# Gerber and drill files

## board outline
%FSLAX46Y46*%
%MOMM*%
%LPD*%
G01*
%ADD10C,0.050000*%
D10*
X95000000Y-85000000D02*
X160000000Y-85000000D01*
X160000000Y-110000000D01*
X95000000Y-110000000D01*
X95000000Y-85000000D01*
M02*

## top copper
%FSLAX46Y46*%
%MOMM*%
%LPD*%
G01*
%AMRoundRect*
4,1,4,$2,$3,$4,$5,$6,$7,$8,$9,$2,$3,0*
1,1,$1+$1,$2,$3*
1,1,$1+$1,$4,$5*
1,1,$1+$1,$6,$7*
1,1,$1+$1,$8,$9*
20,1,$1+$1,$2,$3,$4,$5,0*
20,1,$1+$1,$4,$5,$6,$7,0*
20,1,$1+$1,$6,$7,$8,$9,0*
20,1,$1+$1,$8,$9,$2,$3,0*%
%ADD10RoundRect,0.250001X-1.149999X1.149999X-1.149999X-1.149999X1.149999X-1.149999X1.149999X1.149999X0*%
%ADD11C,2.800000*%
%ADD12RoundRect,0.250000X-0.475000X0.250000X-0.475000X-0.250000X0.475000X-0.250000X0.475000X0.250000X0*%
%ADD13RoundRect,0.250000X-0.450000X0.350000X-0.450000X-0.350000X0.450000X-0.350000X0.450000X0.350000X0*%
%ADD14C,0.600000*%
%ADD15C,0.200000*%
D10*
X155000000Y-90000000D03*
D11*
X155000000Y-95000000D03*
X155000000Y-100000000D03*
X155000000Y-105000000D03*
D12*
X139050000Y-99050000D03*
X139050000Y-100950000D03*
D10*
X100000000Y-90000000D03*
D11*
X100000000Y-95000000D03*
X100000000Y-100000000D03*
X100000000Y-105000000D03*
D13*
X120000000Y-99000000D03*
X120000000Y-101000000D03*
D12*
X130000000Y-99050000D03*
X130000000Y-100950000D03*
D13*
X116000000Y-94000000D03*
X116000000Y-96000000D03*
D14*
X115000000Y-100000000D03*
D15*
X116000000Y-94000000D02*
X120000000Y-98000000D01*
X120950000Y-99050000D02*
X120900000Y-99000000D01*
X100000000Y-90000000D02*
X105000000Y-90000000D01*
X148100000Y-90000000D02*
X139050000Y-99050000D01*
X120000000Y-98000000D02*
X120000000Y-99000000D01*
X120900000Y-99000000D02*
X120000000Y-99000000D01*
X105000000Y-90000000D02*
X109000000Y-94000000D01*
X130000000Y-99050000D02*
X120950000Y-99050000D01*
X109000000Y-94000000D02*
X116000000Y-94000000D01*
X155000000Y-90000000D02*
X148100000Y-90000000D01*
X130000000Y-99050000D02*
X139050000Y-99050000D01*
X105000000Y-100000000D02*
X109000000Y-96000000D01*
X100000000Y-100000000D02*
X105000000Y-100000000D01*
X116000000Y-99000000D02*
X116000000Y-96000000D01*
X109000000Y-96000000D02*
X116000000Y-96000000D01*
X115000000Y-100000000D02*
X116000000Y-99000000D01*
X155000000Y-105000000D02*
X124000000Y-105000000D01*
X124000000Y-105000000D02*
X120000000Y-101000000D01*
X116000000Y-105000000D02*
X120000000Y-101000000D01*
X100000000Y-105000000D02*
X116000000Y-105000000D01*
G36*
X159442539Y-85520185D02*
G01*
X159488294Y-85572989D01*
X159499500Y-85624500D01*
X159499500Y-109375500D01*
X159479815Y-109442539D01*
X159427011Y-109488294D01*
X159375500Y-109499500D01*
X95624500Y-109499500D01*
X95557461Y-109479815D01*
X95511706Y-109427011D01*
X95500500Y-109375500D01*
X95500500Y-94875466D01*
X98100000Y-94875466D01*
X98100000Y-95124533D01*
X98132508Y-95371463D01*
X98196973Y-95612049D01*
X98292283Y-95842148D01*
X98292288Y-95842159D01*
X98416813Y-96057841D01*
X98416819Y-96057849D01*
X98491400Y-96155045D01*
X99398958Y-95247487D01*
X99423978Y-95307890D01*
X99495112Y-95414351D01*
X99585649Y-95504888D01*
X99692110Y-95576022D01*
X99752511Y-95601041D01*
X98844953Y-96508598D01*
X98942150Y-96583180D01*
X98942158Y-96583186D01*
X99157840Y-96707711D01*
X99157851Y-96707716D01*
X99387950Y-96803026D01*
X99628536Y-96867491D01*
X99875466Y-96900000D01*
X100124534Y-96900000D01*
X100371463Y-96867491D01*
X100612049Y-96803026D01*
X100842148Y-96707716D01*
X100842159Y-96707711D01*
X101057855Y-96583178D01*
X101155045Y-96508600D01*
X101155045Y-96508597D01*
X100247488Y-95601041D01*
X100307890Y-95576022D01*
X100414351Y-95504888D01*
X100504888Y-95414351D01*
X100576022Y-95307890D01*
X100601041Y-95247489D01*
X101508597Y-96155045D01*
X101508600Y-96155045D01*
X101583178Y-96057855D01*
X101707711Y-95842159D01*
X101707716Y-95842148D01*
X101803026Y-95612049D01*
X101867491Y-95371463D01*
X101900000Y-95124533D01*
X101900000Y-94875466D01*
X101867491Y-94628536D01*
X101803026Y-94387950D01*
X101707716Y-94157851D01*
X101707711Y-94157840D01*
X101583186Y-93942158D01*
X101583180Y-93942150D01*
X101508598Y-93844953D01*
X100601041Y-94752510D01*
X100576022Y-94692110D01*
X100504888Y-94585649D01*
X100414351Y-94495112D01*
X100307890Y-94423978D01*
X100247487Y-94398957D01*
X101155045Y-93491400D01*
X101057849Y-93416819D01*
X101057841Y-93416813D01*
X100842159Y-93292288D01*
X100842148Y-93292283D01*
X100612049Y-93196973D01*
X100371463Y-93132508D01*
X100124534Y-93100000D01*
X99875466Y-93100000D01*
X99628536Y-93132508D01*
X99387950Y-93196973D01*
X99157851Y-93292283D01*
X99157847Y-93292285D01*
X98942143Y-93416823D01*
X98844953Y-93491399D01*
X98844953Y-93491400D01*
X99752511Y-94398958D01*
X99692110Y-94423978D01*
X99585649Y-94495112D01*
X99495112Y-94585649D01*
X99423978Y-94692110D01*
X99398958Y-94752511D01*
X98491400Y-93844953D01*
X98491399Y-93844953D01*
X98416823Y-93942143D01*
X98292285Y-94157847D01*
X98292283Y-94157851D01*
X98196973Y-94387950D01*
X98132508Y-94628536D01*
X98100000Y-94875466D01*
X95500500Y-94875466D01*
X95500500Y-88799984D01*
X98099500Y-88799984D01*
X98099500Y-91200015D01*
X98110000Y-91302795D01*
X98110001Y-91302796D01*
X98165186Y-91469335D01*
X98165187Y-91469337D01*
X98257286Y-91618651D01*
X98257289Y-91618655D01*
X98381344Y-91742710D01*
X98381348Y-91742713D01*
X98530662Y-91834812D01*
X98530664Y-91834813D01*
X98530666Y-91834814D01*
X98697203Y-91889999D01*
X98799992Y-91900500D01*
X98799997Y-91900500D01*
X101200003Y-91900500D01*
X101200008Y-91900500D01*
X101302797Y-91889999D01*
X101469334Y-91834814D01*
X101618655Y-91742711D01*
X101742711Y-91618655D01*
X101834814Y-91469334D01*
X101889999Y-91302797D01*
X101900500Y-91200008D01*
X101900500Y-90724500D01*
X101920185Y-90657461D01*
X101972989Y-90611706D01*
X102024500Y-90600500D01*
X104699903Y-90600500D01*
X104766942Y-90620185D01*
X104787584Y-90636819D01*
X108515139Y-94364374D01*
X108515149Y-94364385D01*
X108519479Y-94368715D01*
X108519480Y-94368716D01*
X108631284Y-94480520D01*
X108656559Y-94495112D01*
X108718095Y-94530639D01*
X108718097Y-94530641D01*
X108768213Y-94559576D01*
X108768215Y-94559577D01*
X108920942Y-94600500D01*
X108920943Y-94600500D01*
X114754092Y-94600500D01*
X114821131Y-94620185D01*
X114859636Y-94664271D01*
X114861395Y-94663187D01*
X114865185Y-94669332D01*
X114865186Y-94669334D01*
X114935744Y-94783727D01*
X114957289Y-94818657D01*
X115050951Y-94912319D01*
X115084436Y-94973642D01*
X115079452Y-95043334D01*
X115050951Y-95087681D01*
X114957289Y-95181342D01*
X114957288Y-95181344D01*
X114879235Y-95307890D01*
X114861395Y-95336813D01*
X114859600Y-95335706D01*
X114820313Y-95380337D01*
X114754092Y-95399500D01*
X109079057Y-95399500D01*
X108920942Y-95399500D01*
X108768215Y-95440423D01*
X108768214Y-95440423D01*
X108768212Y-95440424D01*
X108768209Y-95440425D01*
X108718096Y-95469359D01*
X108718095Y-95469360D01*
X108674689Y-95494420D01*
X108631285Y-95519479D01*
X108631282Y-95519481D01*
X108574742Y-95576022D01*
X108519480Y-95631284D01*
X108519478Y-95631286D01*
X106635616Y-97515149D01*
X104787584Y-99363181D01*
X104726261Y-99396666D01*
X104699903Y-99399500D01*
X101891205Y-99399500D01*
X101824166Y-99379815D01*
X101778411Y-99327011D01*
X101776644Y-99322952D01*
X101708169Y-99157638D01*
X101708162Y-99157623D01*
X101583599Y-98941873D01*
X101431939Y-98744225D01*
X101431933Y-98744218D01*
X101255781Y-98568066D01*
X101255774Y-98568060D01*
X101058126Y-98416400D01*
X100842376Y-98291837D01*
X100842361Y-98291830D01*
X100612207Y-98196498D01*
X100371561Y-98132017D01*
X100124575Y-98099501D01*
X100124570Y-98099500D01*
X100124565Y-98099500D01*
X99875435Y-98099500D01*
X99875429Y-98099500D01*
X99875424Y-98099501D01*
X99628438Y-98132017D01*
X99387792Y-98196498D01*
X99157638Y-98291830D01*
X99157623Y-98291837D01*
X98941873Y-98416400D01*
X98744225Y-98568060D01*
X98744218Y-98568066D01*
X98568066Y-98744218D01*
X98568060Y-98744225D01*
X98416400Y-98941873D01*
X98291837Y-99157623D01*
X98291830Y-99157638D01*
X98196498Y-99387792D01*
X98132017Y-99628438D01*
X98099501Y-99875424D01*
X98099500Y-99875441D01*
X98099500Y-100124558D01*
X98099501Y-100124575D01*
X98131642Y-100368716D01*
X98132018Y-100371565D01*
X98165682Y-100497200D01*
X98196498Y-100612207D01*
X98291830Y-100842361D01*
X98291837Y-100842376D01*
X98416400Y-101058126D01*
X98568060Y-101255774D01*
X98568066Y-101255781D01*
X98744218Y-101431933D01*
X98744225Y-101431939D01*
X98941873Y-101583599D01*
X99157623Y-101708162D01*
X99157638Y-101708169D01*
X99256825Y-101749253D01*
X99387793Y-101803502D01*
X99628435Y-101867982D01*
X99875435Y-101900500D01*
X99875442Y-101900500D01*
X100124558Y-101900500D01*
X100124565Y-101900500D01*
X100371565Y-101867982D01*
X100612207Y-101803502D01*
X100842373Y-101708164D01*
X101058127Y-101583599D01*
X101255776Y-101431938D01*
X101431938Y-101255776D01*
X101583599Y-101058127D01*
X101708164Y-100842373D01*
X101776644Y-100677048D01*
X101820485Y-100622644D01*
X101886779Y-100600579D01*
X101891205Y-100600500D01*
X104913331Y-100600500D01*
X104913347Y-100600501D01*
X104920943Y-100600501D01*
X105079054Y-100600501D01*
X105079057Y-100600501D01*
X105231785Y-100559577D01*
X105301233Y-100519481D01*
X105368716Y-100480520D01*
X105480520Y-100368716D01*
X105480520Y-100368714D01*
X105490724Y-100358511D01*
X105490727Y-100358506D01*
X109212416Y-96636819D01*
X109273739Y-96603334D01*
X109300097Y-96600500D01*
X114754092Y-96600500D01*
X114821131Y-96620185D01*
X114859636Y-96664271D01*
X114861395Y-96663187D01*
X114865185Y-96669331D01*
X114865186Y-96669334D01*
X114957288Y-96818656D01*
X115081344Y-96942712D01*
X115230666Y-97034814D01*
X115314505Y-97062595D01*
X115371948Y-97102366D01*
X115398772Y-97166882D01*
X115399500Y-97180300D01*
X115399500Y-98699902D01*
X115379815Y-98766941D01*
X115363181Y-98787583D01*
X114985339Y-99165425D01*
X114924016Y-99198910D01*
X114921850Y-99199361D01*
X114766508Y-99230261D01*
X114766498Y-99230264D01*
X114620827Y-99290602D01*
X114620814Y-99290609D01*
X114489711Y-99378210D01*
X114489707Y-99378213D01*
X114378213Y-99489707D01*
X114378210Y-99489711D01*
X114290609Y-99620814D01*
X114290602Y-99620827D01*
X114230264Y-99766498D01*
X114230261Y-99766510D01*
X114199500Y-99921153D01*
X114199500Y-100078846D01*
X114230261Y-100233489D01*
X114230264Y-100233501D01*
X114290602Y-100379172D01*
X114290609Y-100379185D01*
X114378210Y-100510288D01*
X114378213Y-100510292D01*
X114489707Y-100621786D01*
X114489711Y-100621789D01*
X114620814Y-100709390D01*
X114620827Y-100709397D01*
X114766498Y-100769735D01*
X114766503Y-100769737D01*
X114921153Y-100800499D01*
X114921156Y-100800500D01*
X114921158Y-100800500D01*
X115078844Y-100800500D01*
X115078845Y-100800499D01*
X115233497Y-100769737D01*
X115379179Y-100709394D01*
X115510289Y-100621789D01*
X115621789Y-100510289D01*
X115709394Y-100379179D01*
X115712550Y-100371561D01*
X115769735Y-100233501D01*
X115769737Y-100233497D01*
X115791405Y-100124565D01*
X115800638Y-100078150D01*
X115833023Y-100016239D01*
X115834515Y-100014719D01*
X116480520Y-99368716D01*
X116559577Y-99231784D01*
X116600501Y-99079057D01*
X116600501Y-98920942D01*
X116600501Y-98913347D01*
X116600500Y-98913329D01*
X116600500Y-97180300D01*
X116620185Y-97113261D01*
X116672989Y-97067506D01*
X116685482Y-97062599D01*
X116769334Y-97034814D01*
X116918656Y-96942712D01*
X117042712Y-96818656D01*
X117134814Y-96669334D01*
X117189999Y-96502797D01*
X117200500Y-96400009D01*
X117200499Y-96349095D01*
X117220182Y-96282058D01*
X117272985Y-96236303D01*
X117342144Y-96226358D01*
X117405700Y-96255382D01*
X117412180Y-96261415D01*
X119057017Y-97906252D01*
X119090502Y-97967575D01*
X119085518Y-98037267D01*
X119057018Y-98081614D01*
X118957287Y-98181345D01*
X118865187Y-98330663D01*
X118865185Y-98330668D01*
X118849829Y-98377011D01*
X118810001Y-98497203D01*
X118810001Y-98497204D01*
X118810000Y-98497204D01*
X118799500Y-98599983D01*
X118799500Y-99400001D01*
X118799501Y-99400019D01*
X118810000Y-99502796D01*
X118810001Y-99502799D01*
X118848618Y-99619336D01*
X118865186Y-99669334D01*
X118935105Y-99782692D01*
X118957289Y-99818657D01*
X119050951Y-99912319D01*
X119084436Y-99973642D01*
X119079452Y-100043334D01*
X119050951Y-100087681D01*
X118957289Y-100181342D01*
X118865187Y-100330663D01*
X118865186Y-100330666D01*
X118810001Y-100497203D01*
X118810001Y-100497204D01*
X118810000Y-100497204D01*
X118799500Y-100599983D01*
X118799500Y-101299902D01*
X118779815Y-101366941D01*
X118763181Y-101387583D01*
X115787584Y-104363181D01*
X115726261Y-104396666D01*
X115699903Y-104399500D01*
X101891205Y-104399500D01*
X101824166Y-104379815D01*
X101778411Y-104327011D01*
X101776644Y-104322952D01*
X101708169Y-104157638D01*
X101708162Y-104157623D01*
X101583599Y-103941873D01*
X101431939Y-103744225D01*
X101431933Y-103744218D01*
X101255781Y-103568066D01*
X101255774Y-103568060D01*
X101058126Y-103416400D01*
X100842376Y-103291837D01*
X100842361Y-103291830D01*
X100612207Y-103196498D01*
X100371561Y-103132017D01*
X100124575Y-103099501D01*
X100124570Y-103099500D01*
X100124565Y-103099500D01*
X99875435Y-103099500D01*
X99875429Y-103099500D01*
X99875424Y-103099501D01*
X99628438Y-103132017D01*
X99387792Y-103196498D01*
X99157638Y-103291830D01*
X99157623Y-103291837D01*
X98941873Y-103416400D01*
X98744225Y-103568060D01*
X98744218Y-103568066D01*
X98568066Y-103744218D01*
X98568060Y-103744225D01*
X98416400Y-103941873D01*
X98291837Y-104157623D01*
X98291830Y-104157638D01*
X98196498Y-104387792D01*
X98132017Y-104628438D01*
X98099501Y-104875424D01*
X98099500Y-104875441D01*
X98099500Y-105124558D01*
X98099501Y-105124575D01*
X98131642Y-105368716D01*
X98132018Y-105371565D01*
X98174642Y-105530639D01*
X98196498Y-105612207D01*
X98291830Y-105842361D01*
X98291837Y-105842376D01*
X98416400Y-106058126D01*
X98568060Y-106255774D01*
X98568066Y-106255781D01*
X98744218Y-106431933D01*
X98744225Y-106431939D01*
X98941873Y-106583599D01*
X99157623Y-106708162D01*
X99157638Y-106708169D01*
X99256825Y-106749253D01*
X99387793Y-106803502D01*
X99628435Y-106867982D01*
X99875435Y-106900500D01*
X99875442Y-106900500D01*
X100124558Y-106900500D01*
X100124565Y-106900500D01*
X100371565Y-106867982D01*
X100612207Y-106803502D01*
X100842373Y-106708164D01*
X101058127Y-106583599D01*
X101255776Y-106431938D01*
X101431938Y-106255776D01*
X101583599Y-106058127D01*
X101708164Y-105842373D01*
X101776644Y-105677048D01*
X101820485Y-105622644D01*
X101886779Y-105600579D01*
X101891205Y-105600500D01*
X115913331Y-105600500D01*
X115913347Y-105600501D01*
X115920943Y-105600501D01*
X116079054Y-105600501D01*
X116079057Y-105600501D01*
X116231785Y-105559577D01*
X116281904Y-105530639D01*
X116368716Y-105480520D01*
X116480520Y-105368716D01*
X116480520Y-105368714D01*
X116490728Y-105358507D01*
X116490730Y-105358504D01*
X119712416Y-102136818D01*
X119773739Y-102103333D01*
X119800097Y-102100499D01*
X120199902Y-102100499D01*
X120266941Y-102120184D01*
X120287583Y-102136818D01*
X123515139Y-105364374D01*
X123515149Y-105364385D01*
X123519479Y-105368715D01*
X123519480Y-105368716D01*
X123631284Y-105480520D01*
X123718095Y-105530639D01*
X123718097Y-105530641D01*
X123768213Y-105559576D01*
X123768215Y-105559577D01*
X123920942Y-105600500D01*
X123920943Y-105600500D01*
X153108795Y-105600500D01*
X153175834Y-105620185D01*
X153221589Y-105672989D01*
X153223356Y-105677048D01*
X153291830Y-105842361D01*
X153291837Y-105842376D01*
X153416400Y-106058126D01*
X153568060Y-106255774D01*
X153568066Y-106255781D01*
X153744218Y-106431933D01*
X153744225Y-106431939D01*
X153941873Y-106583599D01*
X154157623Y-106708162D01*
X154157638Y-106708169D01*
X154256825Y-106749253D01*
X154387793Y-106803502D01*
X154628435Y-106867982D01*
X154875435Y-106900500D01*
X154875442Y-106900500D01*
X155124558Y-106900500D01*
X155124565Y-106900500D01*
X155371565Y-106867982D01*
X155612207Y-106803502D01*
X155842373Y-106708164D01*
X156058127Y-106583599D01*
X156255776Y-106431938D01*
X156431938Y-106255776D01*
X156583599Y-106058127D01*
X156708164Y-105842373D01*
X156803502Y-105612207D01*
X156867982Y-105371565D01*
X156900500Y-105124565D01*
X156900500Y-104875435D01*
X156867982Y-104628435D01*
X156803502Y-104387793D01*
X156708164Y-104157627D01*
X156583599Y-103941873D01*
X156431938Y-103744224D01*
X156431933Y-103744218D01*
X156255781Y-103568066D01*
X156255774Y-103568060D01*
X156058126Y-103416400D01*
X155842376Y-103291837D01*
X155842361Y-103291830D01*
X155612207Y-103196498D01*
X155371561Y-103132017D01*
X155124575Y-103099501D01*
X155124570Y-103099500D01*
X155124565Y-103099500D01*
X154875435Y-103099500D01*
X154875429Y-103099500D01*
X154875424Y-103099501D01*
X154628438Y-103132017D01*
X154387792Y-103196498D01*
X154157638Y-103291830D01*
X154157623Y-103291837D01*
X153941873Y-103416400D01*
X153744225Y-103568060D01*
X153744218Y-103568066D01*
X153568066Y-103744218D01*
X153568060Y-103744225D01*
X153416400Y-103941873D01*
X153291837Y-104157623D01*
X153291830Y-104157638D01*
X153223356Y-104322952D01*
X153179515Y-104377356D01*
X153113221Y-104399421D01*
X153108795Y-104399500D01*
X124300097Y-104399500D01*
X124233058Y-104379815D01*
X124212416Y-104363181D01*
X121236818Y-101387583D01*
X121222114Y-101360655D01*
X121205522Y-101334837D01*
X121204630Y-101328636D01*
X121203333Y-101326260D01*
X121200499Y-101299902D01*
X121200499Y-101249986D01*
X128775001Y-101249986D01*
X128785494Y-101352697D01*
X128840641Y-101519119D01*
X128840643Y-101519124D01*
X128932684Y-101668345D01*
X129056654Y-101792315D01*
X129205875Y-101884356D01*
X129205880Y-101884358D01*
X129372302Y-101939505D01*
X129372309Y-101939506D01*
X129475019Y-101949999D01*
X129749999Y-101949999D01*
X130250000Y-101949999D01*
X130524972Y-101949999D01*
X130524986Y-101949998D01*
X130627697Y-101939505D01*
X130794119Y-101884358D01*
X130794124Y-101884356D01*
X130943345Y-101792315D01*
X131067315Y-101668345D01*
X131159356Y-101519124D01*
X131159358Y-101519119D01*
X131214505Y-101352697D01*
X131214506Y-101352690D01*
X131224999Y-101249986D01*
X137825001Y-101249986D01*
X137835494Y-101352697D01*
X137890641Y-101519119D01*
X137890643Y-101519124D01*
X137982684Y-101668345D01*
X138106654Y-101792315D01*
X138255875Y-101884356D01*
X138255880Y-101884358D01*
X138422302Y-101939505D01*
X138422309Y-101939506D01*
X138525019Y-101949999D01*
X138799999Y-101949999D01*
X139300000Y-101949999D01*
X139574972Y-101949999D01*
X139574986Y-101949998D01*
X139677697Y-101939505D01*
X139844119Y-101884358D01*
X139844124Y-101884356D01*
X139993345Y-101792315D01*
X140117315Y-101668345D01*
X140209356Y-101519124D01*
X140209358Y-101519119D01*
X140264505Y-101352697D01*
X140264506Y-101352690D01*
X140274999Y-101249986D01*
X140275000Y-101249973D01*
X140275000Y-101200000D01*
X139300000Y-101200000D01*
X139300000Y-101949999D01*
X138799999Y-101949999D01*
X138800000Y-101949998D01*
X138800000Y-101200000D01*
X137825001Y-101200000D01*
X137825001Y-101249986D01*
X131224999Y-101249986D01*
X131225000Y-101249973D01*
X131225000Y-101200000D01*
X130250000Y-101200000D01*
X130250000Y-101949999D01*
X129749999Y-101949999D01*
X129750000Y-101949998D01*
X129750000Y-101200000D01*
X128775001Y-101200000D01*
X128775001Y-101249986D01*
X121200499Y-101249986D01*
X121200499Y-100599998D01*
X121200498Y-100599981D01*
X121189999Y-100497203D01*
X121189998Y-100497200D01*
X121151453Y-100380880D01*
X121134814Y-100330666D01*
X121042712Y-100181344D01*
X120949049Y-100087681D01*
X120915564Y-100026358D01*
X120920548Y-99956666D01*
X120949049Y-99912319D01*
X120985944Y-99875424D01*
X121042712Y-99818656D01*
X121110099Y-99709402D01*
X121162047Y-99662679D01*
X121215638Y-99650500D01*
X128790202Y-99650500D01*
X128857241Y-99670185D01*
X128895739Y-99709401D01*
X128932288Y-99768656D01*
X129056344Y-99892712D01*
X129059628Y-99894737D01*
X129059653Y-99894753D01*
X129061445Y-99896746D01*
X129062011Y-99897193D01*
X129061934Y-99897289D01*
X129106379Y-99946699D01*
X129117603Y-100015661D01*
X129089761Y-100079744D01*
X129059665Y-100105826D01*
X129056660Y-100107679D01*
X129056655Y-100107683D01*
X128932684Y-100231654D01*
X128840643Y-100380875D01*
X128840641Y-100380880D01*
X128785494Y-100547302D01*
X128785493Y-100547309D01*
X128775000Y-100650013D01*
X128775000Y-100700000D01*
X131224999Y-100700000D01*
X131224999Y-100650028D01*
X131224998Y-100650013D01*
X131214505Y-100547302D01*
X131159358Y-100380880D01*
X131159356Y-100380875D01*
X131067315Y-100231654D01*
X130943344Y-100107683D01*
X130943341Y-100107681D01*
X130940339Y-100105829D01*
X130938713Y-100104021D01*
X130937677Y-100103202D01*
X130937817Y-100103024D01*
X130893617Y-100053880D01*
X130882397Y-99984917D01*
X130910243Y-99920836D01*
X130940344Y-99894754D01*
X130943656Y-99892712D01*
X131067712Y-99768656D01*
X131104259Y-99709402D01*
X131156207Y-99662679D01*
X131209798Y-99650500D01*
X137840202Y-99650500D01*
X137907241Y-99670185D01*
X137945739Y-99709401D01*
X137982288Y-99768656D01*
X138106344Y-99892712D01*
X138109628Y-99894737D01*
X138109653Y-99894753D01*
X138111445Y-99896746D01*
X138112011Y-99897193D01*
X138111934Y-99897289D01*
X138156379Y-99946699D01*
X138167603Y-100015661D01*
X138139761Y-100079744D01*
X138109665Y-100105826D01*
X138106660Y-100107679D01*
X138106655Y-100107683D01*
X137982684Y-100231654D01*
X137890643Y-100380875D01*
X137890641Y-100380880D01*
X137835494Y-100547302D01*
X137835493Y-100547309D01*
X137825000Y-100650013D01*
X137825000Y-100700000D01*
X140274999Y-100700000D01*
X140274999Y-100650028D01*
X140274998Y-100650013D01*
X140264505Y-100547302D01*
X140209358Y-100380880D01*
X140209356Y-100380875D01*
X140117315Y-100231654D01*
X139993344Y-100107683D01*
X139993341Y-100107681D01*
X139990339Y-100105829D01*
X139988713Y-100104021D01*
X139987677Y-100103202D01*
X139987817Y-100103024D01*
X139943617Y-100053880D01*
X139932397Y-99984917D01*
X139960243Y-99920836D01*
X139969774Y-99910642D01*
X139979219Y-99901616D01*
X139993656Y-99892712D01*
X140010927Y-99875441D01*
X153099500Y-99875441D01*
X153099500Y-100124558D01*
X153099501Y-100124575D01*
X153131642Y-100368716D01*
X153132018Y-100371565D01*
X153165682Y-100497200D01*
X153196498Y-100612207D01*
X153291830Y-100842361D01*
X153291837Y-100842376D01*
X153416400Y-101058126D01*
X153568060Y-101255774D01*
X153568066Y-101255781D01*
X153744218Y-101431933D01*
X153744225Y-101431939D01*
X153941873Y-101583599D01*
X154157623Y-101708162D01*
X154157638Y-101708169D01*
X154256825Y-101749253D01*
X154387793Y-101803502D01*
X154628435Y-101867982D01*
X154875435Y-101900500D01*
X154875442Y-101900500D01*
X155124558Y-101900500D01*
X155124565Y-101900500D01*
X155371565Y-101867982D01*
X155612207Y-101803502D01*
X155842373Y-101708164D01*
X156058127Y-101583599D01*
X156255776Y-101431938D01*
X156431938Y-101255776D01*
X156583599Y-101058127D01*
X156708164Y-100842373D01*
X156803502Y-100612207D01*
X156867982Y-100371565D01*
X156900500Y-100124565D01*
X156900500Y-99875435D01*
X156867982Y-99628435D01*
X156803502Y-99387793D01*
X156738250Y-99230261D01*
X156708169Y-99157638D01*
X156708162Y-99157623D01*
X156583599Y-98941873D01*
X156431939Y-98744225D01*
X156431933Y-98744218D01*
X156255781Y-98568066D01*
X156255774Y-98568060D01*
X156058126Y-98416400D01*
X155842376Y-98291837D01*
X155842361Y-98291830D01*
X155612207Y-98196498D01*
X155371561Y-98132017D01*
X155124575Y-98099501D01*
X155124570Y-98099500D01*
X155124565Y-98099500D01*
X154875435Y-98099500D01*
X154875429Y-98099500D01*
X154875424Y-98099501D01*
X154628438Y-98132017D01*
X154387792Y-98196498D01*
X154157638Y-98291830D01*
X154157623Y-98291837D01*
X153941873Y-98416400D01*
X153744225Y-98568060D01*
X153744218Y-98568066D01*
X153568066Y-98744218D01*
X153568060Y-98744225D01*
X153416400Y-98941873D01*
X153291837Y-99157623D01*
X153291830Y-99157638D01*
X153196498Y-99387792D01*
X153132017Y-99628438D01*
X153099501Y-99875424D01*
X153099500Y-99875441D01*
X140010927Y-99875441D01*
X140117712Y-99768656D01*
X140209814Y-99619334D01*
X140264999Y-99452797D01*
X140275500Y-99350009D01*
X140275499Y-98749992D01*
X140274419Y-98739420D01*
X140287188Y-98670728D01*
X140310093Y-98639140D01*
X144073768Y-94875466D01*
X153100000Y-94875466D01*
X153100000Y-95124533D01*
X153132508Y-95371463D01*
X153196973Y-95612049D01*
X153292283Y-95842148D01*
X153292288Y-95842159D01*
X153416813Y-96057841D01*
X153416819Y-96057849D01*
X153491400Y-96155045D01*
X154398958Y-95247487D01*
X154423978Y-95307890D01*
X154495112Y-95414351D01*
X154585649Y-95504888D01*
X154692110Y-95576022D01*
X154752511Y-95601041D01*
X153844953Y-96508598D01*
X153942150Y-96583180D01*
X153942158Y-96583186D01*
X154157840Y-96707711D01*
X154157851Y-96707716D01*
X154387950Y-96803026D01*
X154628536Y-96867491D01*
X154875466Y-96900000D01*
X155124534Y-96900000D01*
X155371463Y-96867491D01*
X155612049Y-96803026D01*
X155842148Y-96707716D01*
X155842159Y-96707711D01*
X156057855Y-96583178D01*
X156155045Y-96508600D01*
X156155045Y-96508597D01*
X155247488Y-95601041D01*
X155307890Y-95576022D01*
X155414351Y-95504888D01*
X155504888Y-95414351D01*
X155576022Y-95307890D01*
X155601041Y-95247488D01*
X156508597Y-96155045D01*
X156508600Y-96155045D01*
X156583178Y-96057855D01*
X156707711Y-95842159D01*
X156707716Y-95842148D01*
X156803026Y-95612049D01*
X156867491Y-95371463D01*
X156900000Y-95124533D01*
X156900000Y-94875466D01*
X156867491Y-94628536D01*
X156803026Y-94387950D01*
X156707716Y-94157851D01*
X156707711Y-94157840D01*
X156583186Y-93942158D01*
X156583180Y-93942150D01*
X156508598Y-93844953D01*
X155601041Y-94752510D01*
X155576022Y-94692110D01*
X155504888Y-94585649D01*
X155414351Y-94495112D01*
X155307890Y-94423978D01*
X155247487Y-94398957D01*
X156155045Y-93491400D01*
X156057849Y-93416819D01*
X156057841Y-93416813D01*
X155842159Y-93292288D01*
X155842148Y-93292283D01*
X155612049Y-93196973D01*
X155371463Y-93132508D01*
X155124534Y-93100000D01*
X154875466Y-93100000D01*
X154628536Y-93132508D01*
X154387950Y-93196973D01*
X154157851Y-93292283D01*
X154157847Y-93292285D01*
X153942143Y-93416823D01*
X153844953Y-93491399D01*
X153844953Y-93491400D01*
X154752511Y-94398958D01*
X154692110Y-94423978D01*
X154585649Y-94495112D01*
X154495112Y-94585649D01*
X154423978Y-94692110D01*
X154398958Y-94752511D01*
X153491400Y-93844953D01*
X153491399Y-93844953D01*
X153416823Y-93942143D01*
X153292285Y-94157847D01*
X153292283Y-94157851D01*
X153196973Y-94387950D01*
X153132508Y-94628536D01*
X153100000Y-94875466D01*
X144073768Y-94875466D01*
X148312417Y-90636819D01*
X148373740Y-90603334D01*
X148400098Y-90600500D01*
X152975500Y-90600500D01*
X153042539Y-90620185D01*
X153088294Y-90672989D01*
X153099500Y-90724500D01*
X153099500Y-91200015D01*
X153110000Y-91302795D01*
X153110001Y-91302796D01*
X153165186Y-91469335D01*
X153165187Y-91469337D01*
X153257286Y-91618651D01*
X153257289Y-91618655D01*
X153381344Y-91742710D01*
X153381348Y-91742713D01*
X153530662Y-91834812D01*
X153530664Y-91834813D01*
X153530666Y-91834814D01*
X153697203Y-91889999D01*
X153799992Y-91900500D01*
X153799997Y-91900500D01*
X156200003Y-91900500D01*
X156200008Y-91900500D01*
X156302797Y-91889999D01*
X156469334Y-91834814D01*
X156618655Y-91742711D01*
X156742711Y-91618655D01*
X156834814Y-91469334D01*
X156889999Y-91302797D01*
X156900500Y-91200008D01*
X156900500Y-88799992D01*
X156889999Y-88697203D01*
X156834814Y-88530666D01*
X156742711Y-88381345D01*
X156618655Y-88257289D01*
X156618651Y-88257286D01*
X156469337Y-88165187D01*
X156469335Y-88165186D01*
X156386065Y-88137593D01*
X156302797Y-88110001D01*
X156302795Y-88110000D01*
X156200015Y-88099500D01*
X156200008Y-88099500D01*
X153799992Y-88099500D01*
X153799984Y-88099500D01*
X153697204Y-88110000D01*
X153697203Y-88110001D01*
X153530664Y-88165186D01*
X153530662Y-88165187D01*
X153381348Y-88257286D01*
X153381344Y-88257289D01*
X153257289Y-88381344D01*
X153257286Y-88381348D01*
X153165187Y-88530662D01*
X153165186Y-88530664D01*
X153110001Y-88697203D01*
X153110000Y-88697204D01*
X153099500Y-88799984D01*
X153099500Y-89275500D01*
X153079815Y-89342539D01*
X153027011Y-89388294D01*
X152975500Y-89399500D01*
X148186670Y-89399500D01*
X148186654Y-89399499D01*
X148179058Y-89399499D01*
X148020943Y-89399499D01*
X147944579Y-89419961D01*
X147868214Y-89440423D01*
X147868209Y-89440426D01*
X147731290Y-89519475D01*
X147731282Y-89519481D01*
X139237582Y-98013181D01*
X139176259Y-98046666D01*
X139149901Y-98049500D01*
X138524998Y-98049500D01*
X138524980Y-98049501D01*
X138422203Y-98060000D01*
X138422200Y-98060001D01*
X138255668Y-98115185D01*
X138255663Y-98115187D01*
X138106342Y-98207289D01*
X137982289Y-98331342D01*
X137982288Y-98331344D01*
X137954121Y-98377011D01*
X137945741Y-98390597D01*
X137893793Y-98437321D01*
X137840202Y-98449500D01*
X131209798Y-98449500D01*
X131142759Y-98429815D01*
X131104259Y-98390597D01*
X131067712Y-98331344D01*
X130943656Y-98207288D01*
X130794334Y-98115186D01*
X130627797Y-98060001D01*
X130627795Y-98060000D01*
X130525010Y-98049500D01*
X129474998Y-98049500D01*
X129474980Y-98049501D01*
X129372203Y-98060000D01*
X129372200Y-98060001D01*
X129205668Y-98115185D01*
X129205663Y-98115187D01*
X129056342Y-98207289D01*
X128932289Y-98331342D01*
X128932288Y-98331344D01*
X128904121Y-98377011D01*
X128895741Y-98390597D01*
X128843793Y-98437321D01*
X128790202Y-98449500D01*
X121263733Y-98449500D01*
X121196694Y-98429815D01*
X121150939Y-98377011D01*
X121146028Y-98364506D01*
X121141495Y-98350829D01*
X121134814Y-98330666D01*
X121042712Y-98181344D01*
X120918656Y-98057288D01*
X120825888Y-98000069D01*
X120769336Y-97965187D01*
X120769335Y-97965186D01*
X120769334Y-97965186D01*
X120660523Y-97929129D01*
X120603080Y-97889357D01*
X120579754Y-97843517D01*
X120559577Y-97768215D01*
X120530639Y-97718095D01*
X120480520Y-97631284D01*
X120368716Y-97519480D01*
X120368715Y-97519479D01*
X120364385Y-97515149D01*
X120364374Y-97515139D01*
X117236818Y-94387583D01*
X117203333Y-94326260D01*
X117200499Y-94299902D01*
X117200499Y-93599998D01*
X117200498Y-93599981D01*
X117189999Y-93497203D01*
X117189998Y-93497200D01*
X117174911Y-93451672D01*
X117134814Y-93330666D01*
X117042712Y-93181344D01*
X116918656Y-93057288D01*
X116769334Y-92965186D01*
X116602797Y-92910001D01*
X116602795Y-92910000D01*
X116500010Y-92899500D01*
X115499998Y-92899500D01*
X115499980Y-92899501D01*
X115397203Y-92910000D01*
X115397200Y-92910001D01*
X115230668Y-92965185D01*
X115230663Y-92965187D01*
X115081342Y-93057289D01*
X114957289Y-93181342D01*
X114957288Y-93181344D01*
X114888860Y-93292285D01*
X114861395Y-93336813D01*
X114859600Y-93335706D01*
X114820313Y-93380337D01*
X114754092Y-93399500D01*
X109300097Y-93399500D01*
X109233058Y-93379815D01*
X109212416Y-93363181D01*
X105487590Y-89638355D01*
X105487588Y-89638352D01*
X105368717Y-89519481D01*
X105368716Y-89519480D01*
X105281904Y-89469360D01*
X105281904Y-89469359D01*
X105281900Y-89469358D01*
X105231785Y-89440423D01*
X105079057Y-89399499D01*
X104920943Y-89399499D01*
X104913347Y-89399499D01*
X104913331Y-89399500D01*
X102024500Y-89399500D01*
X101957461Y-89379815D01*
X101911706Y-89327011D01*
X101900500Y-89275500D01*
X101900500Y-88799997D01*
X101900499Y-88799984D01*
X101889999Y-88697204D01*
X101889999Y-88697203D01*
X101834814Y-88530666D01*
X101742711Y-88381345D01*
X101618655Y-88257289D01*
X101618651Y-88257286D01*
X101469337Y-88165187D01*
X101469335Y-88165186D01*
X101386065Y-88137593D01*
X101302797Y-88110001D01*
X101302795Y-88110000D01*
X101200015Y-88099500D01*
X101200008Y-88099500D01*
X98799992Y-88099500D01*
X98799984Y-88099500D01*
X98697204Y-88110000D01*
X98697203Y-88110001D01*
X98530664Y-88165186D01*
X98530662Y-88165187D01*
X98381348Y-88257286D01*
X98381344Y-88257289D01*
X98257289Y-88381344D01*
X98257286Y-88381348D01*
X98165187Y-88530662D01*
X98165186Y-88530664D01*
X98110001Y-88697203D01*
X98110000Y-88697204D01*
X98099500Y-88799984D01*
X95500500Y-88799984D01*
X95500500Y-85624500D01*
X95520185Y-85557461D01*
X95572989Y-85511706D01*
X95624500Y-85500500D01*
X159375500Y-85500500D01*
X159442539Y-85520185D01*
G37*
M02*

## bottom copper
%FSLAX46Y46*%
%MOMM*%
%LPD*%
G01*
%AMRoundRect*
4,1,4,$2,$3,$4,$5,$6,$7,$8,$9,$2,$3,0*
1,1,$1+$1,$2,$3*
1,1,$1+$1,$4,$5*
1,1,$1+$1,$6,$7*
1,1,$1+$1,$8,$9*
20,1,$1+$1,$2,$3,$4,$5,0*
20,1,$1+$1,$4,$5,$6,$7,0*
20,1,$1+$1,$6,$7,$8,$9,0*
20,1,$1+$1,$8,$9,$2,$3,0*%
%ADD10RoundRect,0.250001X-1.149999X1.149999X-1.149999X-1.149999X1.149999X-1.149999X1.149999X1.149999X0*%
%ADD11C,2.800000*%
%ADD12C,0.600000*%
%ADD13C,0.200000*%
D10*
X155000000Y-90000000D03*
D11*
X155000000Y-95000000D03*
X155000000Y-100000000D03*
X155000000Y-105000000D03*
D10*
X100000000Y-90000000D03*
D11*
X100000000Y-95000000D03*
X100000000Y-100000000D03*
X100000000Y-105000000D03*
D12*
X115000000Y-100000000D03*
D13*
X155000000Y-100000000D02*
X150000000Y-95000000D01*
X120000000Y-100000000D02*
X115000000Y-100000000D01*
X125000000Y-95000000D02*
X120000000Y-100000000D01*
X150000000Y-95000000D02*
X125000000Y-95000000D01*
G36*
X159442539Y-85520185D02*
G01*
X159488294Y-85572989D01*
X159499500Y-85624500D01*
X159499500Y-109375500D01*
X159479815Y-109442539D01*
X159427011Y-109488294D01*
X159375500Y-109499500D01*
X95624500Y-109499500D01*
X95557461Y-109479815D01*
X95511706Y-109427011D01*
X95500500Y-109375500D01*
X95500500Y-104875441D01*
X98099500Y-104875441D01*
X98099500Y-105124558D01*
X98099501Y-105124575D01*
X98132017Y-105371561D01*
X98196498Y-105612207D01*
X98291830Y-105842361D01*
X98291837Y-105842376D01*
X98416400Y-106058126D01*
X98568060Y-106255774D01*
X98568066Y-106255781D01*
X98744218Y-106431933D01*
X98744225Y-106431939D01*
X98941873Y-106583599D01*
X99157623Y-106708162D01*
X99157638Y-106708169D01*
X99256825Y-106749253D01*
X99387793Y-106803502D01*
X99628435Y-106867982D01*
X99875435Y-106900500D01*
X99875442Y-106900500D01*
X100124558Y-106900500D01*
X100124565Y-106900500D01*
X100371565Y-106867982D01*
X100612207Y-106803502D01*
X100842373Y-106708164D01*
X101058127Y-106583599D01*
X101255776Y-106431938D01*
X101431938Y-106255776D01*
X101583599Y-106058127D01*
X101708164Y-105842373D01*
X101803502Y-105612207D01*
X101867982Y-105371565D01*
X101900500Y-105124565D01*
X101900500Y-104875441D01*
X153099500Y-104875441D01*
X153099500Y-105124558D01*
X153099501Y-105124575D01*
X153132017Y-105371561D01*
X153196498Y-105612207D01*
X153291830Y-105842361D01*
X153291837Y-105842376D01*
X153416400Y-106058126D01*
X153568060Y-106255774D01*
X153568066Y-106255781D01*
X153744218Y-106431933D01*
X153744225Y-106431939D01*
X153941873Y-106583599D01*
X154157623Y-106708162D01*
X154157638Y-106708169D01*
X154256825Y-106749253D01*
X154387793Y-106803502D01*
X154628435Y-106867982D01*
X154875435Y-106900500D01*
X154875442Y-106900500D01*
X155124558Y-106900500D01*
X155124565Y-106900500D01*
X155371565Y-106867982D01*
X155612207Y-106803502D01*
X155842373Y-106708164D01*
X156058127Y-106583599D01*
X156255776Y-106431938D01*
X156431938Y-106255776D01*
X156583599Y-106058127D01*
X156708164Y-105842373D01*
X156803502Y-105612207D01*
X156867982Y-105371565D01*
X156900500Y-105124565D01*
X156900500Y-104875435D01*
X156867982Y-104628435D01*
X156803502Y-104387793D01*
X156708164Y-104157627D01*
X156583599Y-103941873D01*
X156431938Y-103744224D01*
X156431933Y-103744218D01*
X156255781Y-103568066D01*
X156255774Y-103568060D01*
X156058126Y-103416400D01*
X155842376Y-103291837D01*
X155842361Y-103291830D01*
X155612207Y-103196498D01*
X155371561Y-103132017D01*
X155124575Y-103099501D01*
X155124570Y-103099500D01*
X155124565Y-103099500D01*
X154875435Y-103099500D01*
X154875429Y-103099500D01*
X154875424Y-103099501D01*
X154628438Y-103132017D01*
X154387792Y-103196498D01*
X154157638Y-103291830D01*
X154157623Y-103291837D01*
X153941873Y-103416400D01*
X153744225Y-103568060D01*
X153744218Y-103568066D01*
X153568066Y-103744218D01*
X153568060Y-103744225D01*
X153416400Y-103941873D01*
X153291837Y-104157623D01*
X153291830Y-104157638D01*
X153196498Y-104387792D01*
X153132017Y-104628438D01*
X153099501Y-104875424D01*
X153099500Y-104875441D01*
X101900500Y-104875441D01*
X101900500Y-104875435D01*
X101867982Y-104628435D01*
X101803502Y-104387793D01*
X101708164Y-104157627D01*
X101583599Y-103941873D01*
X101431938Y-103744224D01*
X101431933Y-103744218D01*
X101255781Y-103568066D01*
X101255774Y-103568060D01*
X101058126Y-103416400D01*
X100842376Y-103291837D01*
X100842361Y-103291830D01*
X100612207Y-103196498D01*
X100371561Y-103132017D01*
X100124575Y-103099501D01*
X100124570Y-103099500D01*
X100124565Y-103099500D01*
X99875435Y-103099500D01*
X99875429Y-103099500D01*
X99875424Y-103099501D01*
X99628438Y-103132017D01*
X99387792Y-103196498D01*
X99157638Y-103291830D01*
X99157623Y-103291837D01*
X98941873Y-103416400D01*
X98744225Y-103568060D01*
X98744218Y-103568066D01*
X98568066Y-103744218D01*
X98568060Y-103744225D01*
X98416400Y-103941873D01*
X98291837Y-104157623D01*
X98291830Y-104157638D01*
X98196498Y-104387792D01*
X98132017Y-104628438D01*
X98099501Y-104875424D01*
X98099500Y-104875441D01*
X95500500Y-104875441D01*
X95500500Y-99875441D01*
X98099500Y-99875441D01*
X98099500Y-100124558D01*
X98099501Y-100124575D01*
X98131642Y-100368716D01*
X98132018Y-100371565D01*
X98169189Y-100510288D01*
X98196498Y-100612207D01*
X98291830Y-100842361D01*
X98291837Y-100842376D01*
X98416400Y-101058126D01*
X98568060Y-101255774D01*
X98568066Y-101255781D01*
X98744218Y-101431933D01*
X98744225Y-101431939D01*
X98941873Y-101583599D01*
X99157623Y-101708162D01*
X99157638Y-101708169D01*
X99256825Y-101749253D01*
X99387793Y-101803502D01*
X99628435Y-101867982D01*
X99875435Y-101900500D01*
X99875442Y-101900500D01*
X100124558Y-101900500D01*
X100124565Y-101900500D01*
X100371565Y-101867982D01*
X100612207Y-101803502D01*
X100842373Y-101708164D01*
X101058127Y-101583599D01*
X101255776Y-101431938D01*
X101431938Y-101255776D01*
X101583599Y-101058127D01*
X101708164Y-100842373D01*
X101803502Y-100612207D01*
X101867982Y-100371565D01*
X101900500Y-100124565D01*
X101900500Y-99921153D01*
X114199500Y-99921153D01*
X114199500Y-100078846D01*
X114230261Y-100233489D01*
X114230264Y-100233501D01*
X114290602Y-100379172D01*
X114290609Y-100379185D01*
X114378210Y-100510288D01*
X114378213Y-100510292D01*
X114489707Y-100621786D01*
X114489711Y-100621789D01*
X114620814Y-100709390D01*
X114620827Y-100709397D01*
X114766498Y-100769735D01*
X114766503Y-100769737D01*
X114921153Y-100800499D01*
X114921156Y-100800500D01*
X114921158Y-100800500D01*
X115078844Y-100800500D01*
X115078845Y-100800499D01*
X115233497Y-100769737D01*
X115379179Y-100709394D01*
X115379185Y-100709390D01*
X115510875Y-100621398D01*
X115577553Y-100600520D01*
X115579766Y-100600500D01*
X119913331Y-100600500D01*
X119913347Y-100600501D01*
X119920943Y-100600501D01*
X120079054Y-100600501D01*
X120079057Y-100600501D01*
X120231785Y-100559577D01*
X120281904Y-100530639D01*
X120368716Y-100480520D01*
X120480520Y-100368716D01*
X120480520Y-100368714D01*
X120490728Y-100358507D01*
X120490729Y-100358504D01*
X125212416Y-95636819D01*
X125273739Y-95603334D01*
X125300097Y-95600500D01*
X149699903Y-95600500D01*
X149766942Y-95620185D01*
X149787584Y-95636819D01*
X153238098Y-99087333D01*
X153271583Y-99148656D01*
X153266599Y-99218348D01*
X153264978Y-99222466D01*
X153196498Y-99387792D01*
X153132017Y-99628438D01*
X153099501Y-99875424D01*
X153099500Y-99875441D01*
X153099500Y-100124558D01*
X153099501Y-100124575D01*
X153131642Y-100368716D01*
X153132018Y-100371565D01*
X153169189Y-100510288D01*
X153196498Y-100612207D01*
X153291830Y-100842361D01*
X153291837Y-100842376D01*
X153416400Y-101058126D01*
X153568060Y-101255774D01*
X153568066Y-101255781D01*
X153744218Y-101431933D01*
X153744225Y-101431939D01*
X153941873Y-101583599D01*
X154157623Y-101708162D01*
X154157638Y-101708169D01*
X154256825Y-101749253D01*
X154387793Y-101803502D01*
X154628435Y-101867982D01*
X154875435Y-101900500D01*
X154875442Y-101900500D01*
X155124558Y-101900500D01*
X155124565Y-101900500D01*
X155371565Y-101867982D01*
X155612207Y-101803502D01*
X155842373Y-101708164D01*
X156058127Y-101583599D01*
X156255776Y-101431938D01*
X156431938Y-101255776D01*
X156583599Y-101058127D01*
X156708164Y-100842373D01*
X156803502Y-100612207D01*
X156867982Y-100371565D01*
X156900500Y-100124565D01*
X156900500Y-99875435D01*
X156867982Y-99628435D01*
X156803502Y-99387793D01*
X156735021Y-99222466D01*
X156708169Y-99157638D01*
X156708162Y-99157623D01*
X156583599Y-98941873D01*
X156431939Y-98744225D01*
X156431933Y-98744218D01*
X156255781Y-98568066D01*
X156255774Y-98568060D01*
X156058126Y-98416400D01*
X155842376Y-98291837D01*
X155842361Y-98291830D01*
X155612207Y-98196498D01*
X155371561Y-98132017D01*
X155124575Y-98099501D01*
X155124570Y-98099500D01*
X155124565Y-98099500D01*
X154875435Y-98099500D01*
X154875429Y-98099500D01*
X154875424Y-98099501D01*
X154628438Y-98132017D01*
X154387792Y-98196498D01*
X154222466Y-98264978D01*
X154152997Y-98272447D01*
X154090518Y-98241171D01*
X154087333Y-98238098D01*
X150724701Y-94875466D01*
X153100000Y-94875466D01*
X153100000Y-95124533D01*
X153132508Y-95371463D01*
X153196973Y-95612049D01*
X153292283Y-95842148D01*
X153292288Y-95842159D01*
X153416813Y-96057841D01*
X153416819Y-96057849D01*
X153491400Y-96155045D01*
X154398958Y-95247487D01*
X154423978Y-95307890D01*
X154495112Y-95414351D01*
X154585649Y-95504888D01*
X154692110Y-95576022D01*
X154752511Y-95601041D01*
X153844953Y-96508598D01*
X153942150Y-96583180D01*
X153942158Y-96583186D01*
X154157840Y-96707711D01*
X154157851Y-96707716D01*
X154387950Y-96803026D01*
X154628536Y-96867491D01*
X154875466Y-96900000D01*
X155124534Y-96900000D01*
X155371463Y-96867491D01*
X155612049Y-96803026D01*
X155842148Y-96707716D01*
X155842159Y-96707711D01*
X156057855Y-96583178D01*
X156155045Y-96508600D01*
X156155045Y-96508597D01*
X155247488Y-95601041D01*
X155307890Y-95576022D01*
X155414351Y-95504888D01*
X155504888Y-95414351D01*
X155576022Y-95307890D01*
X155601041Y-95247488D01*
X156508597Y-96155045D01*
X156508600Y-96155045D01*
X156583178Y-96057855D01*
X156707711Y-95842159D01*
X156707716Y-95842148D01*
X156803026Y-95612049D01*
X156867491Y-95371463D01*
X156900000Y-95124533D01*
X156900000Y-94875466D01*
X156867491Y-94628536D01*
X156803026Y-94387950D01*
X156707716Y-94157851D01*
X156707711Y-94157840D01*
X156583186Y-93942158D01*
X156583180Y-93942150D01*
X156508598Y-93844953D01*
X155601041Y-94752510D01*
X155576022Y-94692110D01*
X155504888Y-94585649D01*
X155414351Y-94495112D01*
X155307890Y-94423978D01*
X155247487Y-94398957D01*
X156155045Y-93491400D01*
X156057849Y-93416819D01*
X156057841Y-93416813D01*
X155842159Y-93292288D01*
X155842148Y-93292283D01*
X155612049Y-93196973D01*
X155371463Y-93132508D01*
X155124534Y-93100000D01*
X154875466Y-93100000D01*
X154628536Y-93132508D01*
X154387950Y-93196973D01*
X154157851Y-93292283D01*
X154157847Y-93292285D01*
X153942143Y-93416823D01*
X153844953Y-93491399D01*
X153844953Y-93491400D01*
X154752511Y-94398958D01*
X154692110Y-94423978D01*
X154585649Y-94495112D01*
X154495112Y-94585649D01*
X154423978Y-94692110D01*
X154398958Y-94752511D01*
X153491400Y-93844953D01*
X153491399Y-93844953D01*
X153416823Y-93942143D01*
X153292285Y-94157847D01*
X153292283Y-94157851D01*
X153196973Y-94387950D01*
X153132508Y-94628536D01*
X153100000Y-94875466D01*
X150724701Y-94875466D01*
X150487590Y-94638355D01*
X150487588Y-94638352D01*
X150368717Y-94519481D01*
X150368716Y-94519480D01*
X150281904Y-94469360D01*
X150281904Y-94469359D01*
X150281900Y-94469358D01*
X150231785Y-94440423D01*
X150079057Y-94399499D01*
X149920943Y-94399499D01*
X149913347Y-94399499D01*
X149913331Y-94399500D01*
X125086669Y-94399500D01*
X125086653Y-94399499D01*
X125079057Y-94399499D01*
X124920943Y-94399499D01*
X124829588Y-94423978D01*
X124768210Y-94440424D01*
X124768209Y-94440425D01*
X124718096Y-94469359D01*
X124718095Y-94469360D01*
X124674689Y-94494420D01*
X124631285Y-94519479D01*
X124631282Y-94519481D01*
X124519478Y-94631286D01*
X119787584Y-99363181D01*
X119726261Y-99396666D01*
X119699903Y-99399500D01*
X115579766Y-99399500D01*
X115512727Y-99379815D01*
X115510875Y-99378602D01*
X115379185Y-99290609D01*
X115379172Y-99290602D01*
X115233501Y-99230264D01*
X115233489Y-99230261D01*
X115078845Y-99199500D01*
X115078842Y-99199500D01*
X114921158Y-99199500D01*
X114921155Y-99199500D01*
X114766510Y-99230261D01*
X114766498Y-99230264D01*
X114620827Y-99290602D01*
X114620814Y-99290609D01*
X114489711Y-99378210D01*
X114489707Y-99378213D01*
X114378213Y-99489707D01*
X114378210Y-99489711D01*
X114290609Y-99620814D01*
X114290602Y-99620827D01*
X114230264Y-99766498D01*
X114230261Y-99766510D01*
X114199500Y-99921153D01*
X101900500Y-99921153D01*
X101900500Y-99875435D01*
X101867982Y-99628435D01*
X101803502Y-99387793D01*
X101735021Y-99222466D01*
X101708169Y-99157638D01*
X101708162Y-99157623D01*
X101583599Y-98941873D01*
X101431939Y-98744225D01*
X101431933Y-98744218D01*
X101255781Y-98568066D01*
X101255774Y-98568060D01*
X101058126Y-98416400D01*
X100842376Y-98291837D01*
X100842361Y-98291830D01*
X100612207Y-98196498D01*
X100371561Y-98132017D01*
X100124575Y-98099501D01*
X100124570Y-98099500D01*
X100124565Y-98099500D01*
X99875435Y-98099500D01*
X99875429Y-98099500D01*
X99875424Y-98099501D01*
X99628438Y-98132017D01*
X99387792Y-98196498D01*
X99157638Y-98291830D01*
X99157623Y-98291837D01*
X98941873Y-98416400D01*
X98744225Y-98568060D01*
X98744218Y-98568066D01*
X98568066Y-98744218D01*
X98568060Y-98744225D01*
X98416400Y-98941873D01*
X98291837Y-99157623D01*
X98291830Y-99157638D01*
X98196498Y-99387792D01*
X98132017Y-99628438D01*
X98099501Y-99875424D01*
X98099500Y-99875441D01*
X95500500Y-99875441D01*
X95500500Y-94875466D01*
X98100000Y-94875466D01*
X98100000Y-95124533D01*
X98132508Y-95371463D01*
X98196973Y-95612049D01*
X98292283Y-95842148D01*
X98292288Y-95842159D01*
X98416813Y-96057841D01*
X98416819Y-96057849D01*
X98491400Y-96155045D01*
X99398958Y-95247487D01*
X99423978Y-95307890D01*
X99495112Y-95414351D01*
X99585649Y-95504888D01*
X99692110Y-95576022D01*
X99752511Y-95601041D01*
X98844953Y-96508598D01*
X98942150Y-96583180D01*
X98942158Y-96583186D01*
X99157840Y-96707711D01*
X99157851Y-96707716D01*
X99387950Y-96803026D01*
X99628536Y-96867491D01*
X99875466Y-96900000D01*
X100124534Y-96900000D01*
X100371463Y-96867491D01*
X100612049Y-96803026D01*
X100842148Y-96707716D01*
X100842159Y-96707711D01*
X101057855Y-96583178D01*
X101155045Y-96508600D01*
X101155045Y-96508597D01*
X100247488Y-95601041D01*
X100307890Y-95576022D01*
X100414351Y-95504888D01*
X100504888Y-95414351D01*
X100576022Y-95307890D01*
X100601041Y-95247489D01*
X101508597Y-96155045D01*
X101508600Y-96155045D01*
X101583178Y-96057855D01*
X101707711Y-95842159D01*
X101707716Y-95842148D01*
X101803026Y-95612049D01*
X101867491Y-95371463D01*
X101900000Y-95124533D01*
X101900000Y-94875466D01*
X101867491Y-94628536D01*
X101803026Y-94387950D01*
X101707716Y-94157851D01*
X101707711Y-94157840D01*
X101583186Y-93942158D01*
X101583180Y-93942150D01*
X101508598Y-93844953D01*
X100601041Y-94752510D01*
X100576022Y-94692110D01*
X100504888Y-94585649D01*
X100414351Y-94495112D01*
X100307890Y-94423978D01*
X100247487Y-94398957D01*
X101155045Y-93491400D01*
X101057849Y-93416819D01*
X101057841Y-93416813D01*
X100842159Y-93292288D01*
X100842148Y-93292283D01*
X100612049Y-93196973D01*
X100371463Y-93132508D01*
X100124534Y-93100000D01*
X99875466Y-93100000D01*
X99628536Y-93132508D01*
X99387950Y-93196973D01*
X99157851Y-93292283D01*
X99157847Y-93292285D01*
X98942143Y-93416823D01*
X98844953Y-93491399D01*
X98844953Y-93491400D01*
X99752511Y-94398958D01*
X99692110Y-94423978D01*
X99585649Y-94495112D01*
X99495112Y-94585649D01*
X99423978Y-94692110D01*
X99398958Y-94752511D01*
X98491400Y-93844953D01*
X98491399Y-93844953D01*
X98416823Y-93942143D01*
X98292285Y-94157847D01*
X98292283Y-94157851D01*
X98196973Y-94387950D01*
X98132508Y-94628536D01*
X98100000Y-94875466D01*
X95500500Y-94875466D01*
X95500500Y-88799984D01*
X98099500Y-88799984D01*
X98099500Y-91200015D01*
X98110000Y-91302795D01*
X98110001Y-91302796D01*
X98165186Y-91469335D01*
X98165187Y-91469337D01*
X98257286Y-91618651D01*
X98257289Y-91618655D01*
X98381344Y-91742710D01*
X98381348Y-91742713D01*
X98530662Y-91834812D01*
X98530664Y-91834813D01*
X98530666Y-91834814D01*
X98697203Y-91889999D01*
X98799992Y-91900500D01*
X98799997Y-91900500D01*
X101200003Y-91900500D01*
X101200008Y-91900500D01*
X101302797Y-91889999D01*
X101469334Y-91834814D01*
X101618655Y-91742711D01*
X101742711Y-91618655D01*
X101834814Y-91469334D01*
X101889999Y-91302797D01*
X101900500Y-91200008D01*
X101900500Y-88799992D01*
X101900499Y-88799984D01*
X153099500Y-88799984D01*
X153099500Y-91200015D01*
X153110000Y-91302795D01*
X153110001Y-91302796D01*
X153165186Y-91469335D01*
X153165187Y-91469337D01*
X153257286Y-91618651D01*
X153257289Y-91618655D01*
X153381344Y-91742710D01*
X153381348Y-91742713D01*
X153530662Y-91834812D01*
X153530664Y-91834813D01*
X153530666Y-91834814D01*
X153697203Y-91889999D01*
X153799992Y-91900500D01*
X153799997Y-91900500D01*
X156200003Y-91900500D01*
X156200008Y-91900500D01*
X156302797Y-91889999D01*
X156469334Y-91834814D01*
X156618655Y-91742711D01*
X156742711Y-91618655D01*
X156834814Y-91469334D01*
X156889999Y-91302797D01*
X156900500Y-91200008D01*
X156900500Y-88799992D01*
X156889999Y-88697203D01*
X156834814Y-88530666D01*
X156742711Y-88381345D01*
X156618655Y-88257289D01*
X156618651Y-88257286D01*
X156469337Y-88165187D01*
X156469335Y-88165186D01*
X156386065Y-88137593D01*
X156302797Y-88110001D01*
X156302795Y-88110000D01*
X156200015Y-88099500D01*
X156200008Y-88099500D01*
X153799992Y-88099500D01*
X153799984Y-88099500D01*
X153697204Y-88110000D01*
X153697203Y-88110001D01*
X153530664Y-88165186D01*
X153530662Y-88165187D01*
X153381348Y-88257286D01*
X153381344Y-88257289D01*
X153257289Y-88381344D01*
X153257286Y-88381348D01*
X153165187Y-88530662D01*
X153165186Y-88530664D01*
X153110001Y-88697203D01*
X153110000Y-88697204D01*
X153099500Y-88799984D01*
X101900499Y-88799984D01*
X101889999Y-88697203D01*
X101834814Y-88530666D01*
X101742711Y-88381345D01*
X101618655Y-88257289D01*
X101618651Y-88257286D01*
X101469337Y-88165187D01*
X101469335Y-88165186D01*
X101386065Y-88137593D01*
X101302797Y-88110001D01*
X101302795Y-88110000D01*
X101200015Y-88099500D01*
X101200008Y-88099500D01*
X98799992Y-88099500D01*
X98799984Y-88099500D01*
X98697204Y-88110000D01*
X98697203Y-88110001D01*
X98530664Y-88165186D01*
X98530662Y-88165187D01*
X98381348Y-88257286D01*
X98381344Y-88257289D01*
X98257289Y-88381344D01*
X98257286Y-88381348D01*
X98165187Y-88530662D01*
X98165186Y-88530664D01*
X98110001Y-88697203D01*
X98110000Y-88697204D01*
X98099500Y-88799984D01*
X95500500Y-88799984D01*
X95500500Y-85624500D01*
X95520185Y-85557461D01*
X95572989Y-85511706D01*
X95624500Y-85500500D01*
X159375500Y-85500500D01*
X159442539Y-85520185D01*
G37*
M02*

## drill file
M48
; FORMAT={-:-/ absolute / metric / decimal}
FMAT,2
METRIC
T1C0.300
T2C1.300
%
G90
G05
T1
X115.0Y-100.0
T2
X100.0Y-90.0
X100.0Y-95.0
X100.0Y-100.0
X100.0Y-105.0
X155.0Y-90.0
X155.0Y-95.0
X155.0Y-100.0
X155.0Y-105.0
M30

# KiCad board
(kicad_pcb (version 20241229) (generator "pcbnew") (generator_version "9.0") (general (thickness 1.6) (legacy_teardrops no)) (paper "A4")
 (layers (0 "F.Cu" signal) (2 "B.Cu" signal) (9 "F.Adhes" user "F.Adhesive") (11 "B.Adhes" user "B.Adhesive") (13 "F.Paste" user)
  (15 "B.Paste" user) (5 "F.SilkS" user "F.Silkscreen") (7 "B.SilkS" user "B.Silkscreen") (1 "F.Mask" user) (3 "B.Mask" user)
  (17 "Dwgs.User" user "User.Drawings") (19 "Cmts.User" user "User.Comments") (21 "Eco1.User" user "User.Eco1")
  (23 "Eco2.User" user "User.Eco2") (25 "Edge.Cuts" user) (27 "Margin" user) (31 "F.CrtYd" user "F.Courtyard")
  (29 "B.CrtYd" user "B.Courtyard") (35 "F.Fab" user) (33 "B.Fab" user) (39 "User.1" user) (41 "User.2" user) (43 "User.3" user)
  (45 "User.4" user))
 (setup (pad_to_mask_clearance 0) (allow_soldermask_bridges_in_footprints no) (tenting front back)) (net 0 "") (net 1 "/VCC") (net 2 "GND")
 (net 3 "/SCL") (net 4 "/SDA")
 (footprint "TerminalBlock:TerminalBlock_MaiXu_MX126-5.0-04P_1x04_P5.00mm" (layer "F.Cu") (at 155 90 -90)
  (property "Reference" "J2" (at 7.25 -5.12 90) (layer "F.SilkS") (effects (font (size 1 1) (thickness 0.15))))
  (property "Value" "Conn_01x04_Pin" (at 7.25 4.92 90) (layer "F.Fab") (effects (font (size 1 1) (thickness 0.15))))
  (pad "1" thru_hole roundrect (at 0 0 270) (size 2.8 2.8) (drill 1.3) (layers "*.Cu" "*.Mask") (remove_unused_layers no)
   (roundrect_rratio 0.089286) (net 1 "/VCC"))
  (pad "2" thru_hole circle (at 5 0 270) (size 2.8 2.8) (drill 1.3) (layers "*.Cu" "*.Mask") (remove_unused_layers no) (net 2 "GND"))
  (pad "3" thru_hole circle (at 10 0 270) (size 2.8 2.8) (drill 1.3) (layers "*.Cu" "*.Mask") (remove_unused_layers no) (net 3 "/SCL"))
  (pad "4" thru_hole circle (at 15 0 270) (size 2.8 2.8) (drill 1.3) (layers "*.Cu" "*.Mask") (remove_unused_layers no) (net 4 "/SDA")))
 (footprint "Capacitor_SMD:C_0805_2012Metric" (layer "F.Cu") (at 139.05 100 -90)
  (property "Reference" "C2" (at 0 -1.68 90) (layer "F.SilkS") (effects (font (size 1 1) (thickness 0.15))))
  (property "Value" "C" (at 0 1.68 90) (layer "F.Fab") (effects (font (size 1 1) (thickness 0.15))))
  (pad "1" smd roundrect (at -0.95 0 270) (size 1 1.45) (layers "F.Cu" "F.Mask" "F.Paste") (roundrect_rratio 0.25) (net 1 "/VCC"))
  (pad "2" smd roundrect (at 0.95 0 270) (size 1 1.45) (layers "F.Cu" "F.Mask" "F.Paste") (roundrect_rratio 0.25) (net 2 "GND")))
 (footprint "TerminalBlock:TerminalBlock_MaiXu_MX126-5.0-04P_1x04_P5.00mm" (layer "F.Cu") (at 100 90 -90)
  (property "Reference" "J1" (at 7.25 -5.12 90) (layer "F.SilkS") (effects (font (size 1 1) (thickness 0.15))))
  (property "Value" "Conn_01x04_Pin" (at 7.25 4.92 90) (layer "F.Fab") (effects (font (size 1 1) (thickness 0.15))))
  (pad "1" thru_hole roundrect (at 0 0 270) (size 2.8 2.8) (drill 1.3) (layers "*.Cu" "*.Mask") (remove_unused_layers no)
   (roundrect_rratio 0.089286) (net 1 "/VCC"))
  (pad "2" thru_hole circle (at 5 0 270) (size 2.8 2.8) (drill 1.3) (layers "*.Cu" "*.Mask") (remove_unused_layers no) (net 2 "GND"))
  (pad "3" thru_hole circle (at 10 0 270) (size 2.8 2.8) (drill 1.3) (layers "*.Cu" "*.Mask") (remove_unused_layers no) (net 3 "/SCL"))
  (pad "4" thru_hole circle (at 15 0 270) (size 2.8 2.8) (drill 1.3) (layers "*.Cu" "*.Mask") (remove_unused_layers no) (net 4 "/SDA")))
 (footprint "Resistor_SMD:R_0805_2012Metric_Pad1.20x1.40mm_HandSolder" (layer "F.Cu") (at 120 100 -90)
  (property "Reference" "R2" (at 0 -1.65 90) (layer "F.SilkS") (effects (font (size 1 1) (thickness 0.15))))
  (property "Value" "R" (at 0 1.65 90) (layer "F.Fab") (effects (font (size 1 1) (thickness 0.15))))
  (pad "1" smd roundrect (at -1 0 270) (size 1.2 1.4) (layers "F.Cu" "F.Mask" "F.Paste") (roundrect_rratio 0.208333) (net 1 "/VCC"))
  (pad "2" smd roundrect (at 1 0 270) (size 1.2 1.4) (layers "F.Cu" "F.Mask" "F.Paste") (roundrect_rratio 0.208333) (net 4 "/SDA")))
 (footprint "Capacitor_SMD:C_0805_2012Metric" (layer "F.Cu") (at 130 100 -90)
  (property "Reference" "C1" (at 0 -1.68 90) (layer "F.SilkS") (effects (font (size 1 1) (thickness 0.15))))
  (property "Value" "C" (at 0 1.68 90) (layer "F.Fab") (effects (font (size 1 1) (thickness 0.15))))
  (pad "1" smd roundrect (at -0.95 0 270) (size 1 1.45) (layers "F.Cu" "F.Mask" "F.Paste") (roundrect_rratio 0.25) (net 1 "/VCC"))
  (pad "2" smd roundrect (at 0.95 0 270) (size 1 1.45) (layers "F.Cu" "F.Mask" "F.Paste") (roundrect_rratio 0.25) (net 2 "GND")))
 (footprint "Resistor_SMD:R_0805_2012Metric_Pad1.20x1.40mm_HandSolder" (layer "F.Cu") (at 116 95 -90)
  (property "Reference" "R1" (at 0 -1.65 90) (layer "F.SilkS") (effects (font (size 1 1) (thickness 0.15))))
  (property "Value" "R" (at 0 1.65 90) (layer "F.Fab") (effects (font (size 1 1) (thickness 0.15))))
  (pad "1" smd roundrect (at -1 0 270) (size 1.2 1.4) (layers "F.Cu" "F.Mask" "F.Paste") (roundrect_rratio 0.208333) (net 1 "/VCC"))
  (pad "2" smd roundrect (at 1 0 270) (size 1.2 1.4) (layers "F.Cu" "F.Mask" "F.Paste") (roundrect_rratio 0.208333) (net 3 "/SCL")))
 (gr_rect (start 95 85) (end 160 110) (stroke (width 0.05) (type default)) (fill no) (layer "Edge.Cuts"))
 (segment (start 116 94) (end 120 98) (width 0.2) (layer "F.Cu") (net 1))
 (segment (start 120.95 99.05) (end 120.9 99) (width 0.2) (layer "F.Cu") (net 1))
 (segment (start 100 90) (end 105 90) (width 0.2) (layer "F.Cu") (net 1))
 (segment (start 148.1 90) (end 139.05 99.05) (width 0.2) (layer "F.Cu") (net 1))
 (segment (start 120 98) (end 120 99) (width 0.2) (layer "F.Cu") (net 1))
 (segment (start 120.9 99) (end 120 99) (width 0.2) (layer "F.Cu") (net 1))
 (segment (start 105 90) (end 109 94) (width 0.2) (layer "F.Cu") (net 1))
 (segment (start 130 99.05) (end 120.95 99.05) (width 0.2) (layer "F.Cu") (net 1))
 (segment (start 109 94) (end 116 94) (width 0.2) (layer "F.Cu") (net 1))
 (segment (start 155 90) (end 148.1 90) (width 0.2) (layer "F.Cu") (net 1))
 (segment (start 130 99.05) (end 139.05 99.05) (width 0.2) (layer "F.Cu") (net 1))
 (segment (start 105 100) (end 109 96) (width 0.2) (layer "F.Cu") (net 3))
 (segment (start 100 100) (end 105 100) (width 0.2) (layer "F.Cu") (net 3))
 (segment (start 116 99) (end 116 96) (width 0.2) (layer "F.Cu") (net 3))
 (segment (start 109 96) (end 116 96) (width 0.2) (layer "F.Cu") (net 3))
 (segment (start 115 100) (end 116 99) (width 0.2) (layer "F.Cu") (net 3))
 (via (at 115 100) (size 0.6) (drill 0.3) (layers "F.Cu" "B.Cu") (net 3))
 (segment (start 155 100) (end 150 95) (width 0.2) (layer "B.Cu") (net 3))
 (segment (start 120 100) (end 115 100) (width 0.2) (layer "B.Cu") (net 3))
 (segment (start 125 95) (end 120 100) (width 0.2) (layer "B.Cu") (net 3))
 (segment (start 150 95) (end 125 95) (width 0.2) (layer "B.Cu") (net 3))
 (segment (start 155 105) (end 124 105) (width 0.2) (layer "F.Cu") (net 4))
 (segment (start 124 105) (end 120 101) (width 0.2) (layer "F.Cu") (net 4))
 (segment (start 116 105) (end 120 101) (width 0.2) (layer "F.Cu") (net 4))
 (segment (start 100 105) (end 116 105) (width 0.2) (layer "F.Cu") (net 4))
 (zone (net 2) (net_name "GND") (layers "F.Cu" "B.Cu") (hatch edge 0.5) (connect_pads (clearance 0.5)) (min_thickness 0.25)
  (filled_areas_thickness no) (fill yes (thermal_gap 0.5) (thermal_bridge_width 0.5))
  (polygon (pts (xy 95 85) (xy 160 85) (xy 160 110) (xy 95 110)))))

